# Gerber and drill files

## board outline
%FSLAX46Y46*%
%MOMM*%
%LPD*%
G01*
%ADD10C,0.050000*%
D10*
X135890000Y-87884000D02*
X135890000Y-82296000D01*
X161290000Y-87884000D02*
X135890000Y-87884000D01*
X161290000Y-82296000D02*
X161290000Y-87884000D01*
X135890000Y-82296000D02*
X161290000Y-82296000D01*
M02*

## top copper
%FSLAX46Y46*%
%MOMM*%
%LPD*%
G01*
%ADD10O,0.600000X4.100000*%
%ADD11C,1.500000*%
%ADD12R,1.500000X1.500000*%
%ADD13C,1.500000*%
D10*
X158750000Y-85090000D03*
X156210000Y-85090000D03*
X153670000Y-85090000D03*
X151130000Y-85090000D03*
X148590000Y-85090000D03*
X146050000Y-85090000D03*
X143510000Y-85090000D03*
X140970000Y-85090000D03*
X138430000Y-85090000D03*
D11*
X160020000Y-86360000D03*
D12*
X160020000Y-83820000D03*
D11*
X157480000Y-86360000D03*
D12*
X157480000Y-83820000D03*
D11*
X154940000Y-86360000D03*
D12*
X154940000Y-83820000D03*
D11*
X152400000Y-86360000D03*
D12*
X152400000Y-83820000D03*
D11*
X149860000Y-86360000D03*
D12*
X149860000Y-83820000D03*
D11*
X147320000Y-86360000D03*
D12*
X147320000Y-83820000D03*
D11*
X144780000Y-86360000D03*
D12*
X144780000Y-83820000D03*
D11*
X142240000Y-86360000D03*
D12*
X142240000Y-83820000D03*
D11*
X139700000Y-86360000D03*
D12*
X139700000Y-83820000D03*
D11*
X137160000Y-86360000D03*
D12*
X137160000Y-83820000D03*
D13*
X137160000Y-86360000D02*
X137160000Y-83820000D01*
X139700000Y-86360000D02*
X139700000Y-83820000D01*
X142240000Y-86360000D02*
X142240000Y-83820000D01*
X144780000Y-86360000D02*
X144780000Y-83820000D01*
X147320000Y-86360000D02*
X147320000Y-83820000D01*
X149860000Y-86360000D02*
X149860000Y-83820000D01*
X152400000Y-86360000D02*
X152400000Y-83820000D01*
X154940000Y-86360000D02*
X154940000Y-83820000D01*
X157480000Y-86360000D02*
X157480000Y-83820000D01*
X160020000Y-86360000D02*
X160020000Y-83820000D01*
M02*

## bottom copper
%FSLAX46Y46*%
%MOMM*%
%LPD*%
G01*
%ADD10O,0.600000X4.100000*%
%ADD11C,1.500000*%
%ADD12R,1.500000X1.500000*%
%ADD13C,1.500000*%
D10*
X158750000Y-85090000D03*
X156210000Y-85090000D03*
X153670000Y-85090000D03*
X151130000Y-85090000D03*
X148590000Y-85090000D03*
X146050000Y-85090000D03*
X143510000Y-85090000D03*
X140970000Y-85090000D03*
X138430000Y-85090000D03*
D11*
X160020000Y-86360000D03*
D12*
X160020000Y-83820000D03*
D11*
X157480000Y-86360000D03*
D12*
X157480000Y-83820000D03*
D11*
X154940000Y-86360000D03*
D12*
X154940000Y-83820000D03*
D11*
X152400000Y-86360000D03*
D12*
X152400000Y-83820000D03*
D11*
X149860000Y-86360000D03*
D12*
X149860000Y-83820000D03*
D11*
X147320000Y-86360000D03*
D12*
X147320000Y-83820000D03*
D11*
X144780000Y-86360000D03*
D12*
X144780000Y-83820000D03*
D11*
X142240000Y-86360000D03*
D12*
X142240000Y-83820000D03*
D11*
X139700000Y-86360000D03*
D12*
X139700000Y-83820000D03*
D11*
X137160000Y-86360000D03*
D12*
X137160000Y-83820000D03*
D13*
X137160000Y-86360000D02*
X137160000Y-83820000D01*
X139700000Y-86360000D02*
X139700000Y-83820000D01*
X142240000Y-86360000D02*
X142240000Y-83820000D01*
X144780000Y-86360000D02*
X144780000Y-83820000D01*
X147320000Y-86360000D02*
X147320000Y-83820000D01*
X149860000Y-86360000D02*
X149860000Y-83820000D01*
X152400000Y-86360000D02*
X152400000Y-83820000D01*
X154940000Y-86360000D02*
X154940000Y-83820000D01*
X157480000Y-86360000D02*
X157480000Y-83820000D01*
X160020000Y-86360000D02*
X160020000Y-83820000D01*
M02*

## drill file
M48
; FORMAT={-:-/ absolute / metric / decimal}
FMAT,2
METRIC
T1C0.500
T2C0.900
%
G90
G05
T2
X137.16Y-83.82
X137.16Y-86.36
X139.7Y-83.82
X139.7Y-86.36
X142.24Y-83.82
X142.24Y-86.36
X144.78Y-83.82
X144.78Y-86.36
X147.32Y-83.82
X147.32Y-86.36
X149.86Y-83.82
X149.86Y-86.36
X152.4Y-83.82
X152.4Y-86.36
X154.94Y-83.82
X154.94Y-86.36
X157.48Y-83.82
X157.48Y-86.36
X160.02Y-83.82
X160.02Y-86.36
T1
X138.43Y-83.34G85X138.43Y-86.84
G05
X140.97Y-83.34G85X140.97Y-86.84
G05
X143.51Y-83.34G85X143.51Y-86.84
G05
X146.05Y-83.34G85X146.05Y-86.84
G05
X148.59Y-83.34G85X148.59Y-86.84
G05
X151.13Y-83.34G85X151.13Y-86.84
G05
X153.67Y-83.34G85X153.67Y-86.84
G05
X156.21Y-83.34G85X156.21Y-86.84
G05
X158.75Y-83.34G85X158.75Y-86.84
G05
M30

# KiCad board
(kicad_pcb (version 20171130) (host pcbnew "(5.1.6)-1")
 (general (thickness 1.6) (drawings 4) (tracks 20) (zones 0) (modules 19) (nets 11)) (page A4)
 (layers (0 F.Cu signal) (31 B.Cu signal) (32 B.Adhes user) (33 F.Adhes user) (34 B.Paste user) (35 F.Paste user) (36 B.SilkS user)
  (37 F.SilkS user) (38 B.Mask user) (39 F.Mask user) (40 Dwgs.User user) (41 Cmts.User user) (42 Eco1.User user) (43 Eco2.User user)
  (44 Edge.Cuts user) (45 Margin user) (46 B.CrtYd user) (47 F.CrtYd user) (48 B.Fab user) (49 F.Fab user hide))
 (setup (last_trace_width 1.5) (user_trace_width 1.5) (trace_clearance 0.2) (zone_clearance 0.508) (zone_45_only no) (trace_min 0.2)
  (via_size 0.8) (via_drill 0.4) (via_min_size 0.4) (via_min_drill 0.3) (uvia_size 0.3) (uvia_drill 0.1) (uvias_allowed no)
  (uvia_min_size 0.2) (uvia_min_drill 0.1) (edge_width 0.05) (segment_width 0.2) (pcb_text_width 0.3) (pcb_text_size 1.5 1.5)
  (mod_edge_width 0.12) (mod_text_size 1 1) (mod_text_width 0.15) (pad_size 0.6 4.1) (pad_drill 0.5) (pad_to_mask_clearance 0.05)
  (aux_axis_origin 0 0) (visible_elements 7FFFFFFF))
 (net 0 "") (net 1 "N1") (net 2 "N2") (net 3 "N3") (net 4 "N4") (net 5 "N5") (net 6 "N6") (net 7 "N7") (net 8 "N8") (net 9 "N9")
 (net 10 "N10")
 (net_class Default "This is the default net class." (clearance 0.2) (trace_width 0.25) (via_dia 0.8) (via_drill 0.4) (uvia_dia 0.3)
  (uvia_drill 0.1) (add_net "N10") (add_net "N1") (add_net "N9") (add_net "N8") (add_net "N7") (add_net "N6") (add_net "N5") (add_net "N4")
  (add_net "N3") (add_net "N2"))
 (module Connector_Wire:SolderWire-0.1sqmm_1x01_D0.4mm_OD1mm (layer F.Cu) (at 158.75 85.09)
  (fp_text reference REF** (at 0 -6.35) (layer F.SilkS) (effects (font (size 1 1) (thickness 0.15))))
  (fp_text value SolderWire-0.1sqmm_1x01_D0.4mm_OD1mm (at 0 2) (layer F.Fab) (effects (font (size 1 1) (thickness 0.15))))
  (pad 1 thru_hole oval (at 0 0) (size 0.6 4.1) (drill oval 0.5 4) (layers *.Cu *.Mask)))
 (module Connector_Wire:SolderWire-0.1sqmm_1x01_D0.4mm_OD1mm (layer F.Cu) (at 156.21 85.09)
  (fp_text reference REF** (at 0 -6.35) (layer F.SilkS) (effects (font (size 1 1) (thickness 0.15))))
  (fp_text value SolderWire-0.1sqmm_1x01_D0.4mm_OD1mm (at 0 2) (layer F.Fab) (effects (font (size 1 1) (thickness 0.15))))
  (pad 1 thru_hole oval (at 0 0) (size 0.6 4.1) (drill oval 0.5 4) (layers *.Cu *.Mask)))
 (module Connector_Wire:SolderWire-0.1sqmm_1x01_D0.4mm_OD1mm (layer F.Cu) (at 153.67 85.09)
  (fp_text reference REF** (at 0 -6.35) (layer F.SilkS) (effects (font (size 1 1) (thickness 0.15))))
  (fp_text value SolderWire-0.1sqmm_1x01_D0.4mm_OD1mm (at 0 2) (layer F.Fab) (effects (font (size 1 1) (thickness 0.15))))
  (pad 1 thru_hole oval (at 0 0) (size 0.6 4.1) (drill oval 0.5 4) (layers *.Cu *.Mask)))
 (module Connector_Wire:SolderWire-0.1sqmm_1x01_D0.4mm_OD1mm (layer F.Cu) (at 151.13 85.09)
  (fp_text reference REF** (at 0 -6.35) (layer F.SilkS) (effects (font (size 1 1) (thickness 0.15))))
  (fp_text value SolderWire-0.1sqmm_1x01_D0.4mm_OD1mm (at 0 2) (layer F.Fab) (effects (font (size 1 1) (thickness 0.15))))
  (pad 1 thru_hole oval (at 0 0) (size 0.6 4.1) (drill oval 0.5 4) (layers *.Cu *.Mask)))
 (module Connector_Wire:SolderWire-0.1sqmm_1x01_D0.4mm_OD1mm (layer F.Cu) (at 148.59 85.09)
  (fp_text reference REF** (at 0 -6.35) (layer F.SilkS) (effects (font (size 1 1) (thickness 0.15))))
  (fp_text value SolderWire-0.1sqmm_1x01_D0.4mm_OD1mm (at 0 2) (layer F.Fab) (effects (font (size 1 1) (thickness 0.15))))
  (pad 1 thru_hole oval (at 0 0) (size 0.6 4.1) (drill oval 0.5 4) (layers *.Cu *.Mask)))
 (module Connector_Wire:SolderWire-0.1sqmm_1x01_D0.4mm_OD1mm (layer F.Cu) (at 146.05 85.09)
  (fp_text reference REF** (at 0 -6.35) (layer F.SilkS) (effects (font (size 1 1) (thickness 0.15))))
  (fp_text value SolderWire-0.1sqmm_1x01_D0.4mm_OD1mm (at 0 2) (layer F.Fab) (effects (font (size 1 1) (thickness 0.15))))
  (pad 1 thru_hole oval (at 0 0) (size 0.6 4.1) (drill oval 0.5 4) (layers *.Cu *.Mask)))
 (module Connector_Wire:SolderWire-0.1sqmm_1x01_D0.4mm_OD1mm (layer F.Cu) (at 143.51 85.09)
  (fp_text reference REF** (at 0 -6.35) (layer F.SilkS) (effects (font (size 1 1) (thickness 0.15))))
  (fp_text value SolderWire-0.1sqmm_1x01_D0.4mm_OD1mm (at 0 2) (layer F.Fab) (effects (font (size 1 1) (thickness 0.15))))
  (pad 1 thru_hole oval (at 0 0) (size 0.6 4.1) (drill oval 0.5 4) (layers *.Cu *.Mask)))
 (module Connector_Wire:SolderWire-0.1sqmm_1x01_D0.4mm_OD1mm (layer F.Cu) (at 140.97 85.09)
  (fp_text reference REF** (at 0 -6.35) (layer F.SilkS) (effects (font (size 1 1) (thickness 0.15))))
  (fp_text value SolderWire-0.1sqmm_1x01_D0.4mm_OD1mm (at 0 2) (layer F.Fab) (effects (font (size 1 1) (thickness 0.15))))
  (pad 1 thru_hole oval (at 0 0) (size 0.6 4.1) (drill oval 0.5 4) (layers *.Cu *.Mask)))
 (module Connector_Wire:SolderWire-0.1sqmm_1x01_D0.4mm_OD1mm (layer F.Cu) (at 138.43 85.09)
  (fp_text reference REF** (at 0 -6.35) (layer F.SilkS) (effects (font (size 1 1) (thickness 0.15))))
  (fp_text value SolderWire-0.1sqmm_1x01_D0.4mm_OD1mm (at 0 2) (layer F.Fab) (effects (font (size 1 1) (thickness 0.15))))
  (pad 1 thru_hole oval (at 0 0) (size 0.6 4.1) (drill oval 0.5 4) (layers *.Cu *.Mask)))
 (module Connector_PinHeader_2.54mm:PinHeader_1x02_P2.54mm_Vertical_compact (layer F.Cu) (at 160.02 83.82)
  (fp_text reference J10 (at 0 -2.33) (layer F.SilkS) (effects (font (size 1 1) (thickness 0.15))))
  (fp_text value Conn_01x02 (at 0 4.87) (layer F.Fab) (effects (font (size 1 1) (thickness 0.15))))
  (pad 2 thru_hole circle (at 0 2.54) (size 1.5 1.5) (drill 0.9) (layers *.Cu *.Mask) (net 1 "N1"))
  (pad 1 thru_hole rect (at 0 0) (size 1.5 1.5) (drill 0.9) (layers *.Cu *.Mask) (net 1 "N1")))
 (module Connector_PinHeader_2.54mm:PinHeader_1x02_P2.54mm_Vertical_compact (layer F.Cu) (at 157.48 83.82)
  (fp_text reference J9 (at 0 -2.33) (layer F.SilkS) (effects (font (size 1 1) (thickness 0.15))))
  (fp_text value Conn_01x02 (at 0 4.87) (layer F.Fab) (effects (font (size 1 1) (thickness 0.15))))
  (pad 2 thru_hole circle (at 0 2.54) (size 1.5 1.5) (drill 0.9) (layers *.Cu *.Mask) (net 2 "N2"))
  (pad 1 thru_hole rect (at 0 0) (size 1.5 1.5) (drill 0.9) (layers *.Cu *.Mask) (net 2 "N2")))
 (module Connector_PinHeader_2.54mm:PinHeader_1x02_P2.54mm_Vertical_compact (layer F.Cu) (at 154.94 83.82)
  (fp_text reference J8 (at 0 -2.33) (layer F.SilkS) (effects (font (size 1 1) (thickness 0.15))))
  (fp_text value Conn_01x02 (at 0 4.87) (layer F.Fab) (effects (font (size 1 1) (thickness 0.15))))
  (pad 2 thru_hole circle (at 0 2.54) (size 1.5 1.5) (drill 0.9) (layers *.Cu *.Mask) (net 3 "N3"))
  (pad 1 thru_hole rect (at 0 0) (size 1.5 1.5) (drill 0.9) (layers *.Cu *.Mask) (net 3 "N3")))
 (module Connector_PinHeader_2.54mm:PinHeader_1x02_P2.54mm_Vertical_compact (layer F.Cu) (at 152.4 83.82)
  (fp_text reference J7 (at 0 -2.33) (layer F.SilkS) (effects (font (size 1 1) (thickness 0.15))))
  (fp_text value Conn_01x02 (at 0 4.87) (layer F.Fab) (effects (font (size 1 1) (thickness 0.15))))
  (pad 2 thru_hole circle (at 0 2.54) (size 1.5 1.5) (drill 0.9) (layers *.Cu *.Mask) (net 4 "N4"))
  (pad 1 thru_hole rect (at 0 0) (size 1.5 1.5) (drill 0.9) (layers *.Cu *.Mask) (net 4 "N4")))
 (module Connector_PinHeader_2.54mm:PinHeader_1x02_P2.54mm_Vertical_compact (layer F.Cu) (at 149.86 83.82)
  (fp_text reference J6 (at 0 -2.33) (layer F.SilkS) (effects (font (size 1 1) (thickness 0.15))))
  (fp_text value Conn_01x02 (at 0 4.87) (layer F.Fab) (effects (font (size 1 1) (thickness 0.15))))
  (pad 2 thru_hole circle (at 0 2.54) (size 1.5 1.5) (drill 0.9) (layers *.Cu *.Mask) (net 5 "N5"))
  (pad 1 thru_hole rect (at 0 0) (size 1.5 1.5) (drill 0.9) (layers *.Cu *.Mask) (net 5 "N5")))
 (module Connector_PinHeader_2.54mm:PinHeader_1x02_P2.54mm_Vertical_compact (layer F.Cu) (at 147.32 83.82)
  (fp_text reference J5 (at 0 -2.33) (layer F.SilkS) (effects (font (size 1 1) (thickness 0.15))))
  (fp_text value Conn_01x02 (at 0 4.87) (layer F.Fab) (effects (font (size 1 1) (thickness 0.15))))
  (pad 2 thru_hole circle (at 0 2.54) (size 1.5 1.5) (drill 0.9) (layers *.Cu *.Mask) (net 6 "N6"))
  (pad 1 thru_hole rect (at 0 0) (size 1.5 1.5) (drill 0.9) (layers *.Cu *.Mask) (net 6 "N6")))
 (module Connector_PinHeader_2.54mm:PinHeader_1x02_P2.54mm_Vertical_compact (layer F.Cu) (at 144.78 83.82)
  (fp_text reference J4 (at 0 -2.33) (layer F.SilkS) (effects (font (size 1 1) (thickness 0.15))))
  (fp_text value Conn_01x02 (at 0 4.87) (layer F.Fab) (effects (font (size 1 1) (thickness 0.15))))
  (pad 2 thru_hole circle (at 0 2.54) (size 1.5 1.5) (drill 0.9) (layers *.Cu *.Mask) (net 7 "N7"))
  (pad 1 thru_hole rect (at 0 0) (size 1.5 1.5) (drill 0.9) (layers *.Cu *.Mask) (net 7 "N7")))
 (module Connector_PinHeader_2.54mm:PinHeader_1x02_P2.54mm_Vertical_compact (layer F.Cu) (at 142.24 83.82)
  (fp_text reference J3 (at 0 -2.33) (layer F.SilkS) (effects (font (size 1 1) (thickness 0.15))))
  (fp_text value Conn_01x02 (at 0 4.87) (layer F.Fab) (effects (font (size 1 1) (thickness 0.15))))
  (pad 2 thru_hole circle (at 0 2.54) (size 1.5 1.5) (drill 0.9) (layers *.Cu *.Mask) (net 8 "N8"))
  (pad 1 thru_hole rect (at 0 0) (size 1.5 1.5) (drill 0.9) (layers *.Cu *.Mask) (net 8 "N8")))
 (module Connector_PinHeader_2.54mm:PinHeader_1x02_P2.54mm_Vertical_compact (layer F.Cu) (at 139.7 83.82)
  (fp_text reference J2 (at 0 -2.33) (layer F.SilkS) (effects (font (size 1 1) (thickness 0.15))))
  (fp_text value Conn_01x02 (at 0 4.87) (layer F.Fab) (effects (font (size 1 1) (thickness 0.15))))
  (pad 2 thru_hole circle (at 0 2.54) (size 1.5 1.5) (drill 0.9) (layers *.Cu *.Mask) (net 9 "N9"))
  (pad 1 thru_hole rect (at 0 0) (size 1.5 1.5) (drill 0.9) (layers *.Cu *.Mask) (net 9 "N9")))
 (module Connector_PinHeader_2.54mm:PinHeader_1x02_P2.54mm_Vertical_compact (layer F.Cu) (at 137.16 83.82)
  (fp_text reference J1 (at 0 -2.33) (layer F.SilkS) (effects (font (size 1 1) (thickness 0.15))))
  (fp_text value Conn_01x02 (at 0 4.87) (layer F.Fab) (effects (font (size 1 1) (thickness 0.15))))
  (pad 2 thru_hole circle (at 0 2.54) (size 1.5 1.5) (drill 0.9) (layers *.Cu *.Mask) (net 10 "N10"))
  (pad 1 thru_hole rect (at 0 0) (size 1.5 1.5) (drill 0.9) (layers *.Cu *.Mask) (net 10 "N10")))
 (gr_line (start 135.89 87.884) (end 135.89 82.296) (layer Edge.Cuts) (width 0.05))
 (gr_line (start 161.29 87.884) (end 135.89 87.884) (layer Edge.Cuts) (width 0.05))
 (gr_line (start 161.29 82.296) (end 161.29 87.884) (layer Edge.Cuts) (width 0.05))
 (gr_line (start 135.89 82.296) (end 161.29 82.296) (layer Edge.Cuts) (width 0.05))
 (segment (start 137.16 86.36) (end 137.16 83.82) (width 1.5) (layer B.Cu) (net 10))
 (segment (start 137.16 86.36) (end 137.16 83.82) (width 1.5) (layer F.Cu) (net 10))
 (segment (start 139.7 86.36) (end 139.7 83.82) (width 1.5) (layer B.Cu) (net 9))
 (segment (start 139.7 86.36) (end 139.7 83.82) (width 1.5) (layer F.Cu) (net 9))
 (segment (start 142.24 86.36) (end 142.24 83.82) (width 1.5) (layer B.Cu) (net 8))
 (segment (start 142.24 86.36) (end 142.24 83.82) (width 1.5) (layer F.Cu) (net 8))
 (segment (start 144.78 86.36) (end 144.78 83.82) (width 1.5) (layer B.Cu) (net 7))
 (segment (start 144.78 86.36) (end 144.78 83.82) (width 1.5) (layer F.Cu) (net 7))
 (segment (start 147.32 86.36) (end 147.32 83.82) (width 1.5) (layer B.Cu) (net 6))
 (segment (start 147.32 86.36) (end 147.32 83.82) (width 1.5) (layer F.Cu) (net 6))
 (segment (start 149.86 86.36) (end 149.86 83.82) (width 1.5) (layer B.Cu) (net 5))
 (segment (start 149.86 86.36) (end 149.86 83.82) (width 1.5) (layer F.Cu) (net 5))
 (segment (start 152.4 86.36) (end 152.4 83.82) (width 1.5) (layer B.Cu) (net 4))
 (segment (start 152.4 86.36) (end 152.4 83.82) (width 1.5) (layer F.Cu) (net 4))
 (segment (start 154.94 86.36) (end 154.94 83.82) (width 1.5) (layer B.Cu) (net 3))
 (segment (start 154.94 86.36) (end 154.94 83.82) (width 1.5) (layer F.Cu) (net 3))
 (segment (start 157.48 86.36) (end 157.48 83.82) (width 1.5) (layer B.Cu) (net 2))
 (segment (start 157.48 86.36) (end 157.48 83.82) (width 1.5) (layer F.Cu) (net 2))
 (segment (start 160.02 86.36) (end 160.02 83.82) (width 1.5) (layer B.Cu) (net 1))
 (segment (start 160.02 86.36) (end 160.02 83.82) (width 1.5) (layer F.Cu) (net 1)))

